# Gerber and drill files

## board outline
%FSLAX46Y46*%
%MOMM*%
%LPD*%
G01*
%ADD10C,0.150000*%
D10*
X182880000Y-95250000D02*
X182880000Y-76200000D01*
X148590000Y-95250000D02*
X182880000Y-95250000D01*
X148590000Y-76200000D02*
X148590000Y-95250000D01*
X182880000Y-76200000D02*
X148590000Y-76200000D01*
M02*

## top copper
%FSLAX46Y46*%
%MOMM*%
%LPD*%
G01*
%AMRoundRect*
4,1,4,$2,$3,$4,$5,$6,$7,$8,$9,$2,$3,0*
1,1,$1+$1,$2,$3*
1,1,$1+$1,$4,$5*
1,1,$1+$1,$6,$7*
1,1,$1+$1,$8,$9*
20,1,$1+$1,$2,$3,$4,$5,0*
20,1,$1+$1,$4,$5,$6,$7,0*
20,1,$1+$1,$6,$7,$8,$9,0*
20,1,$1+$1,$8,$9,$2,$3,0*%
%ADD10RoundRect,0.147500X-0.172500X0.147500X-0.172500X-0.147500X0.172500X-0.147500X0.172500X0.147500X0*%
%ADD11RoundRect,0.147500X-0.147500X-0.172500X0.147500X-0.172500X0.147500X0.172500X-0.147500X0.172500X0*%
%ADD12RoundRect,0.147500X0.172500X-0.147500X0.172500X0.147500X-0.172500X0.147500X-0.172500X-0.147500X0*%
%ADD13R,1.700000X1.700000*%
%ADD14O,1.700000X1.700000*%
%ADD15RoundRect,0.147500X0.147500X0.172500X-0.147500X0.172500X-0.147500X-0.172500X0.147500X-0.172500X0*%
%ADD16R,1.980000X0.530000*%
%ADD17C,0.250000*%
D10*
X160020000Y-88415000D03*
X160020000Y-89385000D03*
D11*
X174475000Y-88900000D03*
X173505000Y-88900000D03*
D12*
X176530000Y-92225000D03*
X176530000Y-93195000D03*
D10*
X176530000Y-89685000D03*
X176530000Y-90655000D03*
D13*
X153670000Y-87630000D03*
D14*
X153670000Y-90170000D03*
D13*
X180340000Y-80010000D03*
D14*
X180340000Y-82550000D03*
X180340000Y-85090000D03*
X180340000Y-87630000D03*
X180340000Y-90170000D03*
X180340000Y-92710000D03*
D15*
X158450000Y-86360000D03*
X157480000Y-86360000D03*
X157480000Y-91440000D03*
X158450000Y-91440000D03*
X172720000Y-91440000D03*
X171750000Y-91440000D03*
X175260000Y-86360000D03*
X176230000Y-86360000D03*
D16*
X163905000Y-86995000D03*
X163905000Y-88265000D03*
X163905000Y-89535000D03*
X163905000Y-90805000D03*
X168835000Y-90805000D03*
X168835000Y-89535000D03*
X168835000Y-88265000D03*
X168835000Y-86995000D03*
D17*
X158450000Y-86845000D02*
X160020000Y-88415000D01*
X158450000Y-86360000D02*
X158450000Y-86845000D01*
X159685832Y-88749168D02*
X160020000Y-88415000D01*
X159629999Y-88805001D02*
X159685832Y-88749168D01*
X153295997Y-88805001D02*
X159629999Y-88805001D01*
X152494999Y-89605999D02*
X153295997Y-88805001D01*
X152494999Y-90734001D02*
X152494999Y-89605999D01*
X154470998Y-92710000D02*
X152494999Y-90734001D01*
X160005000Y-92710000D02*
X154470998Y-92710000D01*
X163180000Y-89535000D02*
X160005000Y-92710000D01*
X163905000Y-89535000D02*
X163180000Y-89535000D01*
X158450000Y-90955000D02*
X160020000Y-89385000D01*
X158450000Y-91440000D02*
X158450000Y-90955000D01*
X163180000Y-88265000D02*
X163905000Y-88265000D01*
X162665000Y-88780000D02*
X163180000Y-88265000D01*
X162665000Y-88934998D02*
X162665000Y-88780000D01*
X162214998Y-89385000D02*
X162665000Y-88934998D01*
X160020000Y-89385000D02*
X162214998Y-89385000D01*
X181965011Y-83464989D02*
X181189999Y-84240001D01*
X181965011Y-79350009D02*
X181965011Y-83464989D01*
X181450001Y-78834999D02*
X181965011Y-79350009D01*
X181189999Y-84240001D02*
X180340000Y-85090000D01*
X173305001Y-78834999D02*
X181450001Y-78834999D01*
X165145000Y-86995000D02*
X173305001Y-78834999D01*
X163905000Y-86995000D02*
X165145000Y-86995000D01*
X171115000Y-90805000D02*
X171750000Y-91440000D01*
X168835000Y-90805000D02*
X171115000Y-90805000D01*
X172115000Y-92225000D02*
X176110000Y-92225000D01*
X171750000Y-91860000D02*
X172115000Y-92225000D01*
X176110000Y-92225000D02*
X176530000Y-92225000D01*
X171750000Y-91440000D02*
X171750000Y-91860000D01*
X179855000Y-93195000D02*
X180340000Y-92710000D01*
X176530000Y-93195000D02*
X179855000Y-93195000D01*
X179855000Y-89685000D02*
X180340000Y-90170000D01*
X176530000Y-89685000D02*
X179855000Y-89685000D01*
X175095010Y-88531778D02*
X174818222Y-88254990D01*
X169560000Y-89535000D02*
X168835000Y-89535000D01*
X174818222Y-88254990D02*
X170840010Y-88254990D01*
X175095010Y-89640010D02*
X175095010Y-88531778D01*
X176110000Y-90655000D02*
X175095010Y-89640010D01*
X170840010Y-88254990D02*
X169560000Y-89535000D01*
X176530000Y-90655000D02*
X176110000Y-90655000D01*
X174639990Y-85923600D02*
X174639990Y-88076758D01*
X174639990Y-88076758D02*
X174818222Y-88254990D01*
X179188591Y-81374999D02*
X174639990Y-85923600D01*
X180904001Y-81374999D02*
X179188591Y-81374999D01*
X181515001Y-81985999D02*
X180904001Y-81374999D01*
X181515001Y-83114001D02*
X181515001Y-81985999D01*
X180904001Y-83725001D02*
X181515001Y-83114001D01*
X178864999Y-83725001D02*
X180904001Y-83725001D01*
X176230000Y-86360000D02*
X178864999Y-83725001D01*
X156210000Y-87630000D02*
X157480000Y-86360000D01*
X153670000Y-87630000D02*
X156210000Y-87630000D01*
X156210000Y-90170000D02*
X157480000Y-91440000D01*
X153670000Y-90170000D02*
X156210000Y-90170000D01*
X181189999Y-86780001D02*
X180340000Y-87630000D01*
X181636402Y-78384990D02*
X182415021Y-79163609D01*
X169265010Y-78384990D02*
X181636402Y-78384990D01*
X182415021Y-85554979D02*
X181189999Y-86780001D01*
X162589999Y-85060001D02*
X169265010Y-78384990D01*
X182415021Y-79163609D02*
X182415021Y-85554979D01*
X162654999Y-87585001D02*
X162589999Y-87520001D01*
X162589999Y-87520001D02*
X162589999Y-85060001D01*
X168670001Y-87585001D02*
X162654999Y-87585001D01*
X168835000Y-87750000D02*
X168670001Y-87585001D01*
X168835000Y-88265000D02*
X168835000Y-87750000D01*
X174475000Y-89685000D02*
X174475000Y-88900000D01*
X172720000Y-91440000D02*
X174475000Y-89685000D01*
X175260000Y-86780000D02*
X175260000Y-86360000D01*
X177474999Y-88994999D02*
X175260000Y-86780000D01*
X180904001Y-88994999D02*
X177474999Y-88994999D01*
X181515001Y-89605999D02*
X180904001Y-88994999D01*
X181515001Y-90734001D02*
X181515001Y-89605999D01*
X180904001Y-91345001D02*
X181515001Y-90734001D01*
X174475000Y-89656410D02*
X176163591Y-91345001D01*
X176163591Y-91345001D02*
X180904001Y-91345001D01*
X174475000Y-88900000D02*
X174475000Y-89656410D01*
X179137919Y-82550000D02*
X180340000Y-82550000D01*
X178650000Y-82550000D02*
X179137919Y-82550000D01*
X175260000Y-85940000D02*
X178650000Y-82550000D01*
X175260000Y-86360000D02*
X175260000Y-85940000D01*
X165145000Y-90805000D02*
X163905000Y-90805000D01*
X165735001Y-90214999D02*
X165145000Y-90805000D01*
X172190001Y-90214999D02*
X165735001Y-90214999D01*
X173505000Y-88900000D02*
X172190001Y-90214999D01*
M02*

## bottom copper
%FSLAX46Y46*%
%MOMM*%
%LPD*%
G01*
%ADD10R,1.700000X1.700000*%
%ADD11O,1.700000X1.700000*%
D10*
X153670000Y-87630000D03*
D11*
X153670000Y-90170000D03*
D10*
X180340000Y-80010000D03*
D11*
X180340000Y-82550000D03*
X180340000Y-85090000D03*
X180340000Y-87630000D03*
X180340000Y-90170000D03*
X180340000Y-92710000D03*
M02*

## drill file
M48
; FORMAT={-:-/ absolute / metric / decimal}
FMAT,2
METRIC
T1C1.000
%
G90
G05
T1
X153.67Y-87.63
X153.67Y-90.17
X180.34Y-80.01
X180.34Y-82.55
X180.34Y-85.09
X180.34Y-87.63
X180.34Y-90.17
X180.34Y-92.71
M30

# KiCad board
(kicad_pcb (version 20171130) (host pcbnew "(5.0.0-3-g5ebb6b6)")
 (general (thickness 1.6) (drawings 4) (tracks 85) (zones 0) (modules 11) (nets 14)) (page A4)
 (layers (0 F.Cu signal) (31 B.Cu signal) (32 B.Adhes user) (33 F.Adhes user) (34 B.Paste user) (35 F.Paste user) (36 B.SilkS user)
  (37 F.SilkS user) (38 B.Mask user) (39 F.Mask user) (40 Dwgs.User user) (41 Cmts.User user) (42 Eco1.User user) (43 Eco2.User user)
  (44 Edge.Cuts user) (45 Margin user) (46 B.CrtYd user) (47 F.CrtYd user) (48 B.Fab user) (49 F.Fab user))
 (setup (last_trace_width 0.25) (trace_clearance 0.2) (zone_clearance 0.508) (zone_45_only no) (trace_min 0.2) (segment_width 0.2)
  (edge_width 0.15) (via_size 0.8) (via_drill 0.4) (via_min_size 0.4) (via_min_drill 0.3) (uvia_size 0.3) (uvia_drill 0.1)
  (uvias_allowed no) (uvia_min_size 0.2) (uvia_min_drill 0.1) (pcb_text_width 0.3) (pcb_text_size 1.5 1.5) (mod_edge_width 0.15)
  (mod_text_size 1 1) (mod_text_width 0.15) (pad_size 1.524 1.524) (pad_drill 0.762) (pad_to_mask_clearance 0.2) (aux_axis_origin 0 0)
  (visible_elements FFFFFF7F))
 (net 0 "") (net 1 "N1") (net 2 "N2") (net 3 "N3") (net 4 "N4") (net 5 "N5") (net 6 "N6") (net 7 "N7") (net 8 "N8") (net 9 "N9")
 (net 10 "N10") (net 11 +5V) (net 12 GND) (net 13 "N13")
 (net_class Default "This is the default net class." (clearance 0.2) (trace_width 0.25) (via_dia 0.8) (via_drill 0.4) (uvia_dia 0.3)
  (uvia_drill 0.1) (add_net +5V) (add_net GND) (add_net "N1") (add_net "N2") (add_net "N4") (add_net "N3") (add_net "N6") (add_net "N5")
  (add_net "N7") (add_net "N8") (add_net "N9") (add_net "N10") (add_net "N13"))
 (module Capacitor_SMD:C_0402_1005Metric (layer F.Cu) (at 160.02 88.9 270)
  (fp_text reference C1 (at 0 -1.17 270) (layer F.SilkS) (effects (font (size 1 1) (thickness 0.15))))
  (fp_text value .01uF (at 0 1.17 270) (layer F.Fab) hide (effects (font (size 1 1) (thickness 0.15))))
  (pad 1 smd roundrect (at -0.485 0 270) (size 0.59 0.64) (layers F.Cu F.Paste F.Mask) (roundrect_rratio 0.25) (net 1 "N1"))
  (pad 2 smd roundrect (at 0.485 0 270) (size 0.59 0.64) (layers F.Cu F.Paste F.Mask) (roundrect_rratio 0.25) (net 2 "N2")))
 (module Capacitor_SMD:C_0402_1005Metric (layer F.Cu) (at 173.99 88.9)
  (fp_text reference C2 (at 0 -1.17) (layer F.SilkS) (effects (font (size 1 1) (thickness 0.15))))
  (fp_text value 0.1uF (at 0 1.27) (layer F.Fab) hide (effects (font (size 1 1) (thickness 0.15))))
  (pad 2 smd roundrect (at 0.485 0) (size 0.59 0.64) (layers F.Cu F.Paste F.Mask) (roundrect_rratio 0.25) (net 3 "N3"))
  (pad 1 smd roundrect (at -0.485 0) (size 0.59 0.64) (layers F.Cu F.Paste F.Mask) (roundrect_rratio 0.25) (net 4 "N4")))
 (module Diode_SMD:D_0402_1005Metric (layer F.Cu) (at 176.53 92.71 90)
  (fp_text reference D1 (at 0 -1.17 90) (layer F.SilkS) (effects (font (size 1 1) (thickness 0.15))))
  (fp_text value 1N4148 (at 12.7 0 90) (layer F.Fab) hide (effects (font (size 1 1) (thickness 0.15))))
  (pad 2 smd roundrect (at 0.485 0 90) (size 0.59 0.64) (layers F.Cu F.Paste F.Mask) (roundrect_rratio 0.25) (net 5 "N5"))
  (pad 1 smd roundrect (at -0.485 0 90) (size 0.59 0.64) (layers F.Cu F.Paste F.Mask) (roundrect_rratio 0.25) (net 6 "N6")))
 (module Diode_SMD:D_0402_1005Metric (layer F.Cu) (at 176.53 90.17 270)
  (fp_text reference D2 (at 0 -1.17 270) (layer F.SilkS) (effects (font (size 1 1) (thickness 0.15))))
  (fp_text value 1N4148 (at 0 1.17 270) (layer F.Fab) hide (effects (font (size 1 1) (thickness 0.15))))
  (pad 1 smd roundrect (at -0.485 0 270) (size 0.59 0.64) (layers F.Cu F.Paste F.Mask) (roundrect_rratio 0.25) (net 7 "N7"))
  (pad 2 smd roundrect (at 0.485 0 270) (size 0.59 0.64) (layers F.Cu F.Paste F.Mask) (roundrect_rratio 0.25) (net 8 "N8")))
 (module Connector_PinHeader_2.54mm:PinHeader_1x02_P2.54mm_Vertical (layer F.Cu) (at 153.67 87.63)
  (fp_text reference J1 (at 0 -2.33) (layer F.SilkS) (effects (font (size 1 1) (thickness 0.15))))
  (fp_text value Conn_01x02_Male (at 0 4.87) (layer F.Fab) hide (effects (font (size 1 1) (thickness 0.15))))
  (pad 1 thru_hole rect (at 0 0) (size 1.7 1.7) (drill 1) (layers *.Cu *.Mask) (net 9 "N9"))
  (pad 2 thru_hole oval (at 0 2.54) (size 1.7 1.7) (drill 1) (layers *.Cu *.Mask) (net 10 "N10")))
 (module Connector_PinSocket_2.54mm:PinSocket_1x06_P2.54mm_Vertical (layer F.Cu) (at 180.34 80.01)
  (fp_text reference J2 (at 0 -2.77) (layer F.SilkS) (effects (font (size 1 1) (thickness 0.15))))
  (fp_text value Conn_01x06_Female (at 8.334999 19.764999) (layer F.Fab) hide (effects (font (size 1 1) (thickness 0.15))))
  (pad 1 thru_hole rect (at 0 0) (size 1.7 1.7) (drill 1) (layers *.Cu *.Mask) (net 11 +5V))
  (pad 2 thru_hole oval (at 0 2.54) (size 1.7 1.7) (drill 1) (layers *.Cu *.Mask) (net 3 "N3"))
  (pad 3 thru_hole oval (at 0 5.08) (size 1.7 1.7) (drill 1) (layers *.Cu *.Mask) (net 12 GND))
  (pad 4 thru_hole oval (at 0 7.62) (size 1.7 1.7) (drill 1) (layers *.Cu *.Mask) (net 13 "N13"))
  (pad 5 thru_hole oval (at 0 10.16) (size 1.7 1.7) (drill 1) (layers *.Cu *.Mask) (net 7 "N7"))
  (pad 6 thru_hole oval (at 0 12.7) (size 1.7 1.7) (drill 1) (layers *.Cu *.Mask) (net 6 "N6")))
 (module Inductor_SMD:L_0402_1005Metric (layer F.Cu) (at 157.965 86.36 180)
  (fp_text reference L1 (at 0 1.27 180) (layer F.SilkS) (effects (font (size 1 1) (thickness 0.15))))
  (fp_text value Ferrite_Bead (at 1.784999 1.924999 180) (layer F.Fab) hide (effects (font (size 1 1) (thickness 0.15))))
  (pad 1 smd roundrect (at -0.485 0 180) (size 0.59 0.64) (layers F.Cu F.Paste F.Mask) (roundrect_rratio 0.25) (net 1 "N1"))
  (pad 2 smd roundrect (at 0.485 0 180) (size 0.59 0.64) (layers F.Cu F.Paste F.Mask) (roundrect_rratio 0.25) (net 9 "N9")))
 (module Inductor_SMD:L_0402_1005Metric (layer F.Cu) (at 157.965 91.44 180)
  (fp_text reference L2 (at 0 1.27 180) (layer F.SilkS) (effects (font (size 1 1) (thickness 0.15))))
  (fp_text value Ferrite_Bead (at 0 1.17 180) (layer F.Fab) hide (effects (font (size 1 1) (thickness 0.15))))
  (pad 2 smd roundrect (at 0.485 0 180) (size 0.59 0.64) (layers F.Cu F.Paste F.Mask) (roundrect_rratio 0.25) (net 10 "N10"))
  (pad 1 smd roundrect (at -0.485 0 180) (size 0.59 0.64) (layers F.Cu F.Paste F.Mask) (roundrect_rratio 0.25) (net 2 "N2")))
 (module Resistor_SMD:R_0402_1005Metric (layer F.Cu) (at 172.235 91.44 180)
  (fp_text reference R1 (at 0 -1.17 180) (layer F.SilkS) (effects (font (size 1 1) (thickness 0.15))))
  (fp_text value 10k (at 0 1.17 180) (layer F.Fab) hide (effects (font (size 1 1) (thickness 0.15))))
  (pad 1 smd roundrect (at -0.485 0 180) (size 0.59 0.64) (layers F.Cu F.Paste F.Mask) (roundrect_rratio 0.25) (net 3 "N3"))
  (pad 2 smd roundrect (at 0.485 0 180) (size 0.59 0.64) (layers F.Cu F.Paste F.Mask) (roundrect_rratio 0.25) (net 5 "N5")))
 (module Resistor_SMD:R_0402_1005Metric (layer F.Cu) (at 175.745 86.36 180)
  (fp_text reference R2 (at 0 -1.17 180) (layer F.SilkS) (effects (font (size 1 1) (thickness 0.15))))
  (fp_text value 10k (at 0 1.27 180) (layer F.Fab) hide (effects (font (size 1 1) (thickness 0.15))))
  (pad 2 smd roundrect (at 0.485 0 180) (size 0.59 0.64) (layers F.Cu F.Paste F.Mask) (roundrect_rratio 0.25) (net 3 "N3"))
  (pad 1 smd roundrect (at -0.485 0 180) (size 0.59 0.64) (layers F.Cu F.Paste F.Mask) (roundrect_rratio 0.25) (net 8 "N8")))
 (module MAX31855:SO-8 (layer F.Cu) (at 166.37 88.9)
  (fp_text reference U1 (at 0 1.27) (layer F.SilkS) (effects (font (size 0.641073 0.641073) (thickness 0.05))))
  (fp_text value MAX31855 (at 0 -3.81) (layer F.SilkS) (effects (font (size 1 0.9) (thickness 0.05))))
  (pad 1 smd rect (at -2.465 -1.905) (size 1.98 0.53) (layers F.Cu F.Paste F.Mask) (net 12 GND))
  (pad 2 smd rect (at -2.465 -0.635) (size 1.98 0.53) (layers F.Cu F.Paste F.Mask) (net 2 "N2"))
  (pad 3 smd rect (at -2.465 0.635) (size 1.98 0.53) (layers F.Cu F.Paste F.Mask) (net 1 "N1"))
  (pad 4 smd rect (at -2.465 1.905) (size 1.98 0.53) (layers F.Cu F.Paste F.Mask) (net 4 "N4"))
  (pad 5 smd rect (at 2.465 1.905) (size 1.98 0.53) (layers F.Cu F.Paste F.Mask) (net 5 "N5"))
  (pad 6 smd rect (at 2.465 0.635) (size 1.98 0.53) (layers F.Cu F.Paste F.Mask) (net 8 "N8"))
  (pad 7 smd rect (at 2.465 -0.635) (size 1.98 0.53) (layers F.Cu F.Paste F.Mask) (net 13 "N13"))
  (pad 8 smd rect (at 2.465 -1.905) (size 1.98 0.53) (layers F.Cu F.Paste F.Mask)))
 (gr_line (start 182.88 95.25) (end 182.88 76.2) (layer Edge.Cuts) (width 0.15))
 (gr_line (start 148.59 95.25) (end 182.88 95.25) (layer Edge.Cuts) (width 0.15))
 (gr_line (start 148.59 76.2) (end 148.59 95.25) (layer Edge.Cuts) (width 0.15))
 (gr_line (start 182.88 76.2) (end 148.59 76.2) (layer Edge.Cuts) (width 0.15))
 (segment (start 158.45 86.845) (end 160.02 88.415) (width 0.25) (layer F.Cu) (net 1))
 (segment (start 158.45 86.36) (end 158.45 86.845) (width 0.25) (layer F.Cu) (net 1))
 (segment (start 159.685832 88.749168) (end 160.02 88.415) (width 0.25) (layer F.Cu) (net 1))
 (segment (start 159.629999 88.805001) (end 159.685832 88.749168) (width 0.25) (layer F.Cu) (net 1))
 (segment (start 153.295997 88.805001) (end 159.629999 88.805001) (width 0.25) (layer F.Cu) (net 1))
 (segment (start 152.494999 89.605999) (end 153.295997 88.805001) (width 0.25) (layer F.Cu) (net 1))
 (segment (start 152.494999 90.734001) (end 152.494999 89.605999) (width 0.25) (layer F.Cu) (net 1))
 (segment (start 154.470998 92.71) (end 152.494999 90.734001) (width 0.25) (layer F.Cu) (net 1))
 (segment (start 160.005 92.71) (end 154.470998 92.71) (width 0.25) (layer F.Cu) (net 1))
 (segment (start 163.18 89.535) (end 160.005 92.71) (width 0.25) (layer F.Cu) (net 1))
 (segment (start 163.905 89.535) (end 163.18 89.535) (width 0.25) (layer F.Cu) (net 1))
 (segment (start 158.45 90.955) (end 160.02 89.385) (width 0.25) (layer F.Cu) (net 2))
 (segment (start 158.45 91.44) (end 158.45 90.955) (width 0.25) (layer F.Cu) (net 2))
 (segment (start 163.18 88.265) (end 163.905 88.265) (width 0.25) (layer F.Cu) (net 2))
 (segment (start 162.665 88.78) (end 163.18 88.265) (width 0.25) (layer F.Cu) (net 2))
 (segment (start 162.665 88.934998) (end 162.665 88.78) (width 0.25) (layer F.Cu) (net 2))
 (segment (start 162.214998 89.385) (end 162.665 88.934998) (width 0.25) (layer F.Cu) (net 2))
 (segment (start 160.02 89.385) (end 162.214998 89.385) (width 0.25) (layer F.Cu) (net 2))
 (segment (start 181.965011 83.464989) (end 181.189999 84.240001) (width 0.25) (layer F.Cu) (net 12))
 (segment (start 181.965011 79.350009) (end 181.965011 83.464989) (width 0.25) (layer F.Cu) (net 12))
 (segment (start 181.450001 78.834999) (end 181.965011 79.350009) (width 0.25) (layer F.Cu) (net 12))
 (segment (start 181.189999 84.240001) (end 180.34 85.09) (width 0.25) (layer F.Cu) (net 12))
 (segment (start 173.305001 78.834999) (end 181.450001 78.834999) (width 0.25) (layer F.Cu) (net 12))
 (segment (start 165.145 86.995) (end 173.305001 78.834999) (width 0.25) (layer F.Cu) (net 12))
 (segment (start 163.905 86.995) (end 165.145 86.995) (width 0.25) (layer F.Cu) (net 12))
 (segment (start 171.115 90.805) (end 171.75 91.44) (width 0.25) (layer F.Cu) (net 5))
 (segment (start 168.835 90.805) (end 171.115 90.805) (width 0.25) (layer F.Cu) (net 5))
 (segment (start 172.115 92.225) (end 176.11 92.225) (width 0.25) (layer F.Cu) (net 5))
 (segment (start 171.75 91.86) (end 172.115 92.225) (width 0.25) (layer F.Cu) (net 5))
 (segment (start 176.11 92.225) (end 176.53 92.225) (width 0.25) (layer F.Cu) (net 5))
 (segment (start 171.75 91.44) (end 171.75 91.86) (width 0.25) (layer F.Cu) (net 5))
 (segment (start 179.855 93.195) (end 180.34 92.71) (width 0.25) (layer F.Cu) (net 6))
 (segment (start 176.53 93.195) (end 179.855 93.195) (width 0.25) (layer F.Cu) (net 6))
 (segment (start 179.855 89.685) (end 180.34 90.17) (width 0.25) (layer F.Cu) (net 7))
 (segment (start 176.53 89.685) (end 179.855 89.685) (width 0.25) (layer F.Cu) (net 7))
 (segment (start 175.09501 88.531778) (end 174.818222 88.25499) (width 0.25) (layer F.Cu) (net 8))
 (segment (start 169.56 89.535) (end 168.835 89.535) (width 0.25) (layer F.Cu) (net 8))
 (segment (start 174.818222 88.25499) (end 170.84001 88.25499) (width 0.25) (layer F.Cu) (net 8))
 (segment (start 175.09501 89.64001) (end 175.09501 88.531778) (width 0.25) (layer F.Cu) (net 8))
 (segment (start 176.11 90.655) (end 175.09501 89.64001) (width 0.25) (layer F.Cu) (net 8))
 (segment (start 170.84001 88.25499) (end 169.56 89.535) (width 0.25) (layer F.Cu) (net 8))
 (segment (start 176.53 90.655) (end 176.11 90.655) (width 0.25) (layer F.Cu) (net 8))
 (segment (start 174.63999 85.9236) (end 174.63999 88.076758) (width 0.25) (layer F.Cu) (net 8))
 (segment (start 174.63999 88.076758) (end 174.818222 88.25499) (width 0.25) (layer F.Cu) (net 8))
 (segment (start 179.188591 81.374999) (end 174.63999 85.9236) (width 0.25) (layer F.Cu) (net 8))
 (segment (start 180.904001 81.374999) (end 179.188591 81.374999) (width 0.25) (layer F.Cu) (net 8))
 (segment (start 181.515001 81.985999) (end 180.904001 81.374999) (width 0.25) (layer F.Cu) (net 8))
 (segment (start 181.515001 83.114001) (end 181.515001 81.985999) (width 0.25) (layer F.Cu) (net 8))
 (segment (start 180.904001 83.725001) (end 181.515001 83.114001) (width 0.25) (layer F.Cu) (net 8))
 (segment (start 178.864999 83.725001) (end 180.904001 83.725001) (width 0.25) (layer F.Cu) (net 8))
 (segment (start 176.23 86.36) (end 178.864999 83.725001) (width 0.25) (layer F.Cu) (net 8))
 (segment (start 156.21 87.63) (end 157.48 86.36) (width 0.25) (layer F.Cu) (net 9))
 (segment (start 153.67 87.63) (end 156.21 87.63) (width 0.25) (layer F.Cu) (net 9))
 (segment (start 156.21 90.17) (end 157.48 91.44) (width 0.25) (layer F.Cu) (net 10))
 (segment (start 153.67 90.17) (end 156.21 90.17) (width 0.25) (layer F.Cu) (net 10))
 (segment (start 181.189999 86.780001) (end 180.34 87.63) (width 0.25) (layer F.Cu) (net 13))
 (segment (start 181.636402 78.38499) (end 182.415021 79.163609) (width 0.25) (layer F.Cu) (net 13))
 (segment (start 169.26501 78.38499) (end 181.636402 78.38499) (width 0.25) (layer F.Cu) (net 13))
 (segment (start 182.415021 85.554979) (end 181.189999 86.780001) (width 0.25) (layer F.Cu) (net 13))
 (segment (start 162.589999 85.060001) (end 169.26501 78.38499) (width 0.25) (layer F.Cu) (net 13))
 (segment (start 182.415021 79.163609) (end 182.415021 85.554979) (width 0.25) (layer F.Cu) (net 13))
 (segment (start 162.654999 87.585001) (end 162.589999 87.520001) (width 0.25) (layer F.Cu) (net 13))
 (segment (start 162.589999 87.520001) (end 162.589999 85.060001) (width 0.25) (layer F.Cu) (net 13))
 (segment (start 168.670001 87.585001) (end 162.654999 87.585001) (width 0.25) (layer F.Cu) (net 13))
 (segment (start 168.835 87.75) (end 168.670001 87.585001) (width 0.25) (layer F.Cu) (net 13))
 (segment (start 168.835 88.265) (end 168.835 87.75) (width 0.25) (layer F.Cu) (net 13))
 (segment (start 174.475 89.685) (end 174.475 88.9) (width 0.25) (layer F.Cu) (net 3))
 (segment (start 172.72 91.44) (end 174.475 89.685) (width 0.25) (layer F.Cu) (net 3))
 (segment (start 175.26 86.78) (end 175.26 86.36) (width 0.25) (layer F.Cu) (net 3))
 (segment (start 177.474999 88.994999) (end 175.26 86.78) (width 0.25) (layer F.Cu) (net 3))
 (segment (start 180.904001 88.994999) (end 177.474999 88.994999) (width 0.25) (layer F.Cu) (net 3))
 (segment (start 181.515001 89.605999) (end 180.904001 88.994999) (width 0.25) (layer F.Cu) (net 3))
 (segment (start 181.515001 90.734001) (end 181.515001 89.605999) (width 0.25) (layer F.Cu) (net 3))
 (segment (start 180.904001 91.345001) (end 181.515001 90.734001) (width 0.25) (layer F.Cu) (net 3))
 (segment (start 174.475 89.65641) (end 176.163591 91.345001) (width 0.25) (layer F.Cu) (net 3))
 (segment (start 176.163591 91.345001) (end 180.904001 91.345001) (width 0.25) (layer F.Cu) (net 3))
 (segment (start 174.475 88.9) (end 174.475 89.65641) (width 0.25) (layer F.Cu) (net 3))
 (segment (start 179.137919 82.55) (end 180.34 82.55) (width 0.25) (layer F.Cu) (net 3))
 (segment (start 178.65 82.55) (end 179.137919 82.55) (width 0.25) (layer F.Cu) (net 3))
 (segment (start 175.26 85.94) (end 178.65 82.55) (width 0.25) (layer F.Cu) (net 3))
 (segment (start 175.26 86.36) (end 175.26 85.94) (width 0.25) (layer F.Cu) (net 3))
 (segment (start 165.145 90.805) (end 163.905 90.805) (width 0.25) (layer F.Cu) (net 4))
 (segment (start 165.735001 90.214999) (end 165.145 90.805) (width 0.25) (layer F.Cu) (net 4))
 (segment (start 172.190001 90.214999) (end 165.735001 90.214999) (width 0.25) (layer F.Cu) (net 4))
 (segment (start 173.505 88.9) (end 172.190001 90.214999) (width 0.25) (layer F.Cu) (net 4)))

